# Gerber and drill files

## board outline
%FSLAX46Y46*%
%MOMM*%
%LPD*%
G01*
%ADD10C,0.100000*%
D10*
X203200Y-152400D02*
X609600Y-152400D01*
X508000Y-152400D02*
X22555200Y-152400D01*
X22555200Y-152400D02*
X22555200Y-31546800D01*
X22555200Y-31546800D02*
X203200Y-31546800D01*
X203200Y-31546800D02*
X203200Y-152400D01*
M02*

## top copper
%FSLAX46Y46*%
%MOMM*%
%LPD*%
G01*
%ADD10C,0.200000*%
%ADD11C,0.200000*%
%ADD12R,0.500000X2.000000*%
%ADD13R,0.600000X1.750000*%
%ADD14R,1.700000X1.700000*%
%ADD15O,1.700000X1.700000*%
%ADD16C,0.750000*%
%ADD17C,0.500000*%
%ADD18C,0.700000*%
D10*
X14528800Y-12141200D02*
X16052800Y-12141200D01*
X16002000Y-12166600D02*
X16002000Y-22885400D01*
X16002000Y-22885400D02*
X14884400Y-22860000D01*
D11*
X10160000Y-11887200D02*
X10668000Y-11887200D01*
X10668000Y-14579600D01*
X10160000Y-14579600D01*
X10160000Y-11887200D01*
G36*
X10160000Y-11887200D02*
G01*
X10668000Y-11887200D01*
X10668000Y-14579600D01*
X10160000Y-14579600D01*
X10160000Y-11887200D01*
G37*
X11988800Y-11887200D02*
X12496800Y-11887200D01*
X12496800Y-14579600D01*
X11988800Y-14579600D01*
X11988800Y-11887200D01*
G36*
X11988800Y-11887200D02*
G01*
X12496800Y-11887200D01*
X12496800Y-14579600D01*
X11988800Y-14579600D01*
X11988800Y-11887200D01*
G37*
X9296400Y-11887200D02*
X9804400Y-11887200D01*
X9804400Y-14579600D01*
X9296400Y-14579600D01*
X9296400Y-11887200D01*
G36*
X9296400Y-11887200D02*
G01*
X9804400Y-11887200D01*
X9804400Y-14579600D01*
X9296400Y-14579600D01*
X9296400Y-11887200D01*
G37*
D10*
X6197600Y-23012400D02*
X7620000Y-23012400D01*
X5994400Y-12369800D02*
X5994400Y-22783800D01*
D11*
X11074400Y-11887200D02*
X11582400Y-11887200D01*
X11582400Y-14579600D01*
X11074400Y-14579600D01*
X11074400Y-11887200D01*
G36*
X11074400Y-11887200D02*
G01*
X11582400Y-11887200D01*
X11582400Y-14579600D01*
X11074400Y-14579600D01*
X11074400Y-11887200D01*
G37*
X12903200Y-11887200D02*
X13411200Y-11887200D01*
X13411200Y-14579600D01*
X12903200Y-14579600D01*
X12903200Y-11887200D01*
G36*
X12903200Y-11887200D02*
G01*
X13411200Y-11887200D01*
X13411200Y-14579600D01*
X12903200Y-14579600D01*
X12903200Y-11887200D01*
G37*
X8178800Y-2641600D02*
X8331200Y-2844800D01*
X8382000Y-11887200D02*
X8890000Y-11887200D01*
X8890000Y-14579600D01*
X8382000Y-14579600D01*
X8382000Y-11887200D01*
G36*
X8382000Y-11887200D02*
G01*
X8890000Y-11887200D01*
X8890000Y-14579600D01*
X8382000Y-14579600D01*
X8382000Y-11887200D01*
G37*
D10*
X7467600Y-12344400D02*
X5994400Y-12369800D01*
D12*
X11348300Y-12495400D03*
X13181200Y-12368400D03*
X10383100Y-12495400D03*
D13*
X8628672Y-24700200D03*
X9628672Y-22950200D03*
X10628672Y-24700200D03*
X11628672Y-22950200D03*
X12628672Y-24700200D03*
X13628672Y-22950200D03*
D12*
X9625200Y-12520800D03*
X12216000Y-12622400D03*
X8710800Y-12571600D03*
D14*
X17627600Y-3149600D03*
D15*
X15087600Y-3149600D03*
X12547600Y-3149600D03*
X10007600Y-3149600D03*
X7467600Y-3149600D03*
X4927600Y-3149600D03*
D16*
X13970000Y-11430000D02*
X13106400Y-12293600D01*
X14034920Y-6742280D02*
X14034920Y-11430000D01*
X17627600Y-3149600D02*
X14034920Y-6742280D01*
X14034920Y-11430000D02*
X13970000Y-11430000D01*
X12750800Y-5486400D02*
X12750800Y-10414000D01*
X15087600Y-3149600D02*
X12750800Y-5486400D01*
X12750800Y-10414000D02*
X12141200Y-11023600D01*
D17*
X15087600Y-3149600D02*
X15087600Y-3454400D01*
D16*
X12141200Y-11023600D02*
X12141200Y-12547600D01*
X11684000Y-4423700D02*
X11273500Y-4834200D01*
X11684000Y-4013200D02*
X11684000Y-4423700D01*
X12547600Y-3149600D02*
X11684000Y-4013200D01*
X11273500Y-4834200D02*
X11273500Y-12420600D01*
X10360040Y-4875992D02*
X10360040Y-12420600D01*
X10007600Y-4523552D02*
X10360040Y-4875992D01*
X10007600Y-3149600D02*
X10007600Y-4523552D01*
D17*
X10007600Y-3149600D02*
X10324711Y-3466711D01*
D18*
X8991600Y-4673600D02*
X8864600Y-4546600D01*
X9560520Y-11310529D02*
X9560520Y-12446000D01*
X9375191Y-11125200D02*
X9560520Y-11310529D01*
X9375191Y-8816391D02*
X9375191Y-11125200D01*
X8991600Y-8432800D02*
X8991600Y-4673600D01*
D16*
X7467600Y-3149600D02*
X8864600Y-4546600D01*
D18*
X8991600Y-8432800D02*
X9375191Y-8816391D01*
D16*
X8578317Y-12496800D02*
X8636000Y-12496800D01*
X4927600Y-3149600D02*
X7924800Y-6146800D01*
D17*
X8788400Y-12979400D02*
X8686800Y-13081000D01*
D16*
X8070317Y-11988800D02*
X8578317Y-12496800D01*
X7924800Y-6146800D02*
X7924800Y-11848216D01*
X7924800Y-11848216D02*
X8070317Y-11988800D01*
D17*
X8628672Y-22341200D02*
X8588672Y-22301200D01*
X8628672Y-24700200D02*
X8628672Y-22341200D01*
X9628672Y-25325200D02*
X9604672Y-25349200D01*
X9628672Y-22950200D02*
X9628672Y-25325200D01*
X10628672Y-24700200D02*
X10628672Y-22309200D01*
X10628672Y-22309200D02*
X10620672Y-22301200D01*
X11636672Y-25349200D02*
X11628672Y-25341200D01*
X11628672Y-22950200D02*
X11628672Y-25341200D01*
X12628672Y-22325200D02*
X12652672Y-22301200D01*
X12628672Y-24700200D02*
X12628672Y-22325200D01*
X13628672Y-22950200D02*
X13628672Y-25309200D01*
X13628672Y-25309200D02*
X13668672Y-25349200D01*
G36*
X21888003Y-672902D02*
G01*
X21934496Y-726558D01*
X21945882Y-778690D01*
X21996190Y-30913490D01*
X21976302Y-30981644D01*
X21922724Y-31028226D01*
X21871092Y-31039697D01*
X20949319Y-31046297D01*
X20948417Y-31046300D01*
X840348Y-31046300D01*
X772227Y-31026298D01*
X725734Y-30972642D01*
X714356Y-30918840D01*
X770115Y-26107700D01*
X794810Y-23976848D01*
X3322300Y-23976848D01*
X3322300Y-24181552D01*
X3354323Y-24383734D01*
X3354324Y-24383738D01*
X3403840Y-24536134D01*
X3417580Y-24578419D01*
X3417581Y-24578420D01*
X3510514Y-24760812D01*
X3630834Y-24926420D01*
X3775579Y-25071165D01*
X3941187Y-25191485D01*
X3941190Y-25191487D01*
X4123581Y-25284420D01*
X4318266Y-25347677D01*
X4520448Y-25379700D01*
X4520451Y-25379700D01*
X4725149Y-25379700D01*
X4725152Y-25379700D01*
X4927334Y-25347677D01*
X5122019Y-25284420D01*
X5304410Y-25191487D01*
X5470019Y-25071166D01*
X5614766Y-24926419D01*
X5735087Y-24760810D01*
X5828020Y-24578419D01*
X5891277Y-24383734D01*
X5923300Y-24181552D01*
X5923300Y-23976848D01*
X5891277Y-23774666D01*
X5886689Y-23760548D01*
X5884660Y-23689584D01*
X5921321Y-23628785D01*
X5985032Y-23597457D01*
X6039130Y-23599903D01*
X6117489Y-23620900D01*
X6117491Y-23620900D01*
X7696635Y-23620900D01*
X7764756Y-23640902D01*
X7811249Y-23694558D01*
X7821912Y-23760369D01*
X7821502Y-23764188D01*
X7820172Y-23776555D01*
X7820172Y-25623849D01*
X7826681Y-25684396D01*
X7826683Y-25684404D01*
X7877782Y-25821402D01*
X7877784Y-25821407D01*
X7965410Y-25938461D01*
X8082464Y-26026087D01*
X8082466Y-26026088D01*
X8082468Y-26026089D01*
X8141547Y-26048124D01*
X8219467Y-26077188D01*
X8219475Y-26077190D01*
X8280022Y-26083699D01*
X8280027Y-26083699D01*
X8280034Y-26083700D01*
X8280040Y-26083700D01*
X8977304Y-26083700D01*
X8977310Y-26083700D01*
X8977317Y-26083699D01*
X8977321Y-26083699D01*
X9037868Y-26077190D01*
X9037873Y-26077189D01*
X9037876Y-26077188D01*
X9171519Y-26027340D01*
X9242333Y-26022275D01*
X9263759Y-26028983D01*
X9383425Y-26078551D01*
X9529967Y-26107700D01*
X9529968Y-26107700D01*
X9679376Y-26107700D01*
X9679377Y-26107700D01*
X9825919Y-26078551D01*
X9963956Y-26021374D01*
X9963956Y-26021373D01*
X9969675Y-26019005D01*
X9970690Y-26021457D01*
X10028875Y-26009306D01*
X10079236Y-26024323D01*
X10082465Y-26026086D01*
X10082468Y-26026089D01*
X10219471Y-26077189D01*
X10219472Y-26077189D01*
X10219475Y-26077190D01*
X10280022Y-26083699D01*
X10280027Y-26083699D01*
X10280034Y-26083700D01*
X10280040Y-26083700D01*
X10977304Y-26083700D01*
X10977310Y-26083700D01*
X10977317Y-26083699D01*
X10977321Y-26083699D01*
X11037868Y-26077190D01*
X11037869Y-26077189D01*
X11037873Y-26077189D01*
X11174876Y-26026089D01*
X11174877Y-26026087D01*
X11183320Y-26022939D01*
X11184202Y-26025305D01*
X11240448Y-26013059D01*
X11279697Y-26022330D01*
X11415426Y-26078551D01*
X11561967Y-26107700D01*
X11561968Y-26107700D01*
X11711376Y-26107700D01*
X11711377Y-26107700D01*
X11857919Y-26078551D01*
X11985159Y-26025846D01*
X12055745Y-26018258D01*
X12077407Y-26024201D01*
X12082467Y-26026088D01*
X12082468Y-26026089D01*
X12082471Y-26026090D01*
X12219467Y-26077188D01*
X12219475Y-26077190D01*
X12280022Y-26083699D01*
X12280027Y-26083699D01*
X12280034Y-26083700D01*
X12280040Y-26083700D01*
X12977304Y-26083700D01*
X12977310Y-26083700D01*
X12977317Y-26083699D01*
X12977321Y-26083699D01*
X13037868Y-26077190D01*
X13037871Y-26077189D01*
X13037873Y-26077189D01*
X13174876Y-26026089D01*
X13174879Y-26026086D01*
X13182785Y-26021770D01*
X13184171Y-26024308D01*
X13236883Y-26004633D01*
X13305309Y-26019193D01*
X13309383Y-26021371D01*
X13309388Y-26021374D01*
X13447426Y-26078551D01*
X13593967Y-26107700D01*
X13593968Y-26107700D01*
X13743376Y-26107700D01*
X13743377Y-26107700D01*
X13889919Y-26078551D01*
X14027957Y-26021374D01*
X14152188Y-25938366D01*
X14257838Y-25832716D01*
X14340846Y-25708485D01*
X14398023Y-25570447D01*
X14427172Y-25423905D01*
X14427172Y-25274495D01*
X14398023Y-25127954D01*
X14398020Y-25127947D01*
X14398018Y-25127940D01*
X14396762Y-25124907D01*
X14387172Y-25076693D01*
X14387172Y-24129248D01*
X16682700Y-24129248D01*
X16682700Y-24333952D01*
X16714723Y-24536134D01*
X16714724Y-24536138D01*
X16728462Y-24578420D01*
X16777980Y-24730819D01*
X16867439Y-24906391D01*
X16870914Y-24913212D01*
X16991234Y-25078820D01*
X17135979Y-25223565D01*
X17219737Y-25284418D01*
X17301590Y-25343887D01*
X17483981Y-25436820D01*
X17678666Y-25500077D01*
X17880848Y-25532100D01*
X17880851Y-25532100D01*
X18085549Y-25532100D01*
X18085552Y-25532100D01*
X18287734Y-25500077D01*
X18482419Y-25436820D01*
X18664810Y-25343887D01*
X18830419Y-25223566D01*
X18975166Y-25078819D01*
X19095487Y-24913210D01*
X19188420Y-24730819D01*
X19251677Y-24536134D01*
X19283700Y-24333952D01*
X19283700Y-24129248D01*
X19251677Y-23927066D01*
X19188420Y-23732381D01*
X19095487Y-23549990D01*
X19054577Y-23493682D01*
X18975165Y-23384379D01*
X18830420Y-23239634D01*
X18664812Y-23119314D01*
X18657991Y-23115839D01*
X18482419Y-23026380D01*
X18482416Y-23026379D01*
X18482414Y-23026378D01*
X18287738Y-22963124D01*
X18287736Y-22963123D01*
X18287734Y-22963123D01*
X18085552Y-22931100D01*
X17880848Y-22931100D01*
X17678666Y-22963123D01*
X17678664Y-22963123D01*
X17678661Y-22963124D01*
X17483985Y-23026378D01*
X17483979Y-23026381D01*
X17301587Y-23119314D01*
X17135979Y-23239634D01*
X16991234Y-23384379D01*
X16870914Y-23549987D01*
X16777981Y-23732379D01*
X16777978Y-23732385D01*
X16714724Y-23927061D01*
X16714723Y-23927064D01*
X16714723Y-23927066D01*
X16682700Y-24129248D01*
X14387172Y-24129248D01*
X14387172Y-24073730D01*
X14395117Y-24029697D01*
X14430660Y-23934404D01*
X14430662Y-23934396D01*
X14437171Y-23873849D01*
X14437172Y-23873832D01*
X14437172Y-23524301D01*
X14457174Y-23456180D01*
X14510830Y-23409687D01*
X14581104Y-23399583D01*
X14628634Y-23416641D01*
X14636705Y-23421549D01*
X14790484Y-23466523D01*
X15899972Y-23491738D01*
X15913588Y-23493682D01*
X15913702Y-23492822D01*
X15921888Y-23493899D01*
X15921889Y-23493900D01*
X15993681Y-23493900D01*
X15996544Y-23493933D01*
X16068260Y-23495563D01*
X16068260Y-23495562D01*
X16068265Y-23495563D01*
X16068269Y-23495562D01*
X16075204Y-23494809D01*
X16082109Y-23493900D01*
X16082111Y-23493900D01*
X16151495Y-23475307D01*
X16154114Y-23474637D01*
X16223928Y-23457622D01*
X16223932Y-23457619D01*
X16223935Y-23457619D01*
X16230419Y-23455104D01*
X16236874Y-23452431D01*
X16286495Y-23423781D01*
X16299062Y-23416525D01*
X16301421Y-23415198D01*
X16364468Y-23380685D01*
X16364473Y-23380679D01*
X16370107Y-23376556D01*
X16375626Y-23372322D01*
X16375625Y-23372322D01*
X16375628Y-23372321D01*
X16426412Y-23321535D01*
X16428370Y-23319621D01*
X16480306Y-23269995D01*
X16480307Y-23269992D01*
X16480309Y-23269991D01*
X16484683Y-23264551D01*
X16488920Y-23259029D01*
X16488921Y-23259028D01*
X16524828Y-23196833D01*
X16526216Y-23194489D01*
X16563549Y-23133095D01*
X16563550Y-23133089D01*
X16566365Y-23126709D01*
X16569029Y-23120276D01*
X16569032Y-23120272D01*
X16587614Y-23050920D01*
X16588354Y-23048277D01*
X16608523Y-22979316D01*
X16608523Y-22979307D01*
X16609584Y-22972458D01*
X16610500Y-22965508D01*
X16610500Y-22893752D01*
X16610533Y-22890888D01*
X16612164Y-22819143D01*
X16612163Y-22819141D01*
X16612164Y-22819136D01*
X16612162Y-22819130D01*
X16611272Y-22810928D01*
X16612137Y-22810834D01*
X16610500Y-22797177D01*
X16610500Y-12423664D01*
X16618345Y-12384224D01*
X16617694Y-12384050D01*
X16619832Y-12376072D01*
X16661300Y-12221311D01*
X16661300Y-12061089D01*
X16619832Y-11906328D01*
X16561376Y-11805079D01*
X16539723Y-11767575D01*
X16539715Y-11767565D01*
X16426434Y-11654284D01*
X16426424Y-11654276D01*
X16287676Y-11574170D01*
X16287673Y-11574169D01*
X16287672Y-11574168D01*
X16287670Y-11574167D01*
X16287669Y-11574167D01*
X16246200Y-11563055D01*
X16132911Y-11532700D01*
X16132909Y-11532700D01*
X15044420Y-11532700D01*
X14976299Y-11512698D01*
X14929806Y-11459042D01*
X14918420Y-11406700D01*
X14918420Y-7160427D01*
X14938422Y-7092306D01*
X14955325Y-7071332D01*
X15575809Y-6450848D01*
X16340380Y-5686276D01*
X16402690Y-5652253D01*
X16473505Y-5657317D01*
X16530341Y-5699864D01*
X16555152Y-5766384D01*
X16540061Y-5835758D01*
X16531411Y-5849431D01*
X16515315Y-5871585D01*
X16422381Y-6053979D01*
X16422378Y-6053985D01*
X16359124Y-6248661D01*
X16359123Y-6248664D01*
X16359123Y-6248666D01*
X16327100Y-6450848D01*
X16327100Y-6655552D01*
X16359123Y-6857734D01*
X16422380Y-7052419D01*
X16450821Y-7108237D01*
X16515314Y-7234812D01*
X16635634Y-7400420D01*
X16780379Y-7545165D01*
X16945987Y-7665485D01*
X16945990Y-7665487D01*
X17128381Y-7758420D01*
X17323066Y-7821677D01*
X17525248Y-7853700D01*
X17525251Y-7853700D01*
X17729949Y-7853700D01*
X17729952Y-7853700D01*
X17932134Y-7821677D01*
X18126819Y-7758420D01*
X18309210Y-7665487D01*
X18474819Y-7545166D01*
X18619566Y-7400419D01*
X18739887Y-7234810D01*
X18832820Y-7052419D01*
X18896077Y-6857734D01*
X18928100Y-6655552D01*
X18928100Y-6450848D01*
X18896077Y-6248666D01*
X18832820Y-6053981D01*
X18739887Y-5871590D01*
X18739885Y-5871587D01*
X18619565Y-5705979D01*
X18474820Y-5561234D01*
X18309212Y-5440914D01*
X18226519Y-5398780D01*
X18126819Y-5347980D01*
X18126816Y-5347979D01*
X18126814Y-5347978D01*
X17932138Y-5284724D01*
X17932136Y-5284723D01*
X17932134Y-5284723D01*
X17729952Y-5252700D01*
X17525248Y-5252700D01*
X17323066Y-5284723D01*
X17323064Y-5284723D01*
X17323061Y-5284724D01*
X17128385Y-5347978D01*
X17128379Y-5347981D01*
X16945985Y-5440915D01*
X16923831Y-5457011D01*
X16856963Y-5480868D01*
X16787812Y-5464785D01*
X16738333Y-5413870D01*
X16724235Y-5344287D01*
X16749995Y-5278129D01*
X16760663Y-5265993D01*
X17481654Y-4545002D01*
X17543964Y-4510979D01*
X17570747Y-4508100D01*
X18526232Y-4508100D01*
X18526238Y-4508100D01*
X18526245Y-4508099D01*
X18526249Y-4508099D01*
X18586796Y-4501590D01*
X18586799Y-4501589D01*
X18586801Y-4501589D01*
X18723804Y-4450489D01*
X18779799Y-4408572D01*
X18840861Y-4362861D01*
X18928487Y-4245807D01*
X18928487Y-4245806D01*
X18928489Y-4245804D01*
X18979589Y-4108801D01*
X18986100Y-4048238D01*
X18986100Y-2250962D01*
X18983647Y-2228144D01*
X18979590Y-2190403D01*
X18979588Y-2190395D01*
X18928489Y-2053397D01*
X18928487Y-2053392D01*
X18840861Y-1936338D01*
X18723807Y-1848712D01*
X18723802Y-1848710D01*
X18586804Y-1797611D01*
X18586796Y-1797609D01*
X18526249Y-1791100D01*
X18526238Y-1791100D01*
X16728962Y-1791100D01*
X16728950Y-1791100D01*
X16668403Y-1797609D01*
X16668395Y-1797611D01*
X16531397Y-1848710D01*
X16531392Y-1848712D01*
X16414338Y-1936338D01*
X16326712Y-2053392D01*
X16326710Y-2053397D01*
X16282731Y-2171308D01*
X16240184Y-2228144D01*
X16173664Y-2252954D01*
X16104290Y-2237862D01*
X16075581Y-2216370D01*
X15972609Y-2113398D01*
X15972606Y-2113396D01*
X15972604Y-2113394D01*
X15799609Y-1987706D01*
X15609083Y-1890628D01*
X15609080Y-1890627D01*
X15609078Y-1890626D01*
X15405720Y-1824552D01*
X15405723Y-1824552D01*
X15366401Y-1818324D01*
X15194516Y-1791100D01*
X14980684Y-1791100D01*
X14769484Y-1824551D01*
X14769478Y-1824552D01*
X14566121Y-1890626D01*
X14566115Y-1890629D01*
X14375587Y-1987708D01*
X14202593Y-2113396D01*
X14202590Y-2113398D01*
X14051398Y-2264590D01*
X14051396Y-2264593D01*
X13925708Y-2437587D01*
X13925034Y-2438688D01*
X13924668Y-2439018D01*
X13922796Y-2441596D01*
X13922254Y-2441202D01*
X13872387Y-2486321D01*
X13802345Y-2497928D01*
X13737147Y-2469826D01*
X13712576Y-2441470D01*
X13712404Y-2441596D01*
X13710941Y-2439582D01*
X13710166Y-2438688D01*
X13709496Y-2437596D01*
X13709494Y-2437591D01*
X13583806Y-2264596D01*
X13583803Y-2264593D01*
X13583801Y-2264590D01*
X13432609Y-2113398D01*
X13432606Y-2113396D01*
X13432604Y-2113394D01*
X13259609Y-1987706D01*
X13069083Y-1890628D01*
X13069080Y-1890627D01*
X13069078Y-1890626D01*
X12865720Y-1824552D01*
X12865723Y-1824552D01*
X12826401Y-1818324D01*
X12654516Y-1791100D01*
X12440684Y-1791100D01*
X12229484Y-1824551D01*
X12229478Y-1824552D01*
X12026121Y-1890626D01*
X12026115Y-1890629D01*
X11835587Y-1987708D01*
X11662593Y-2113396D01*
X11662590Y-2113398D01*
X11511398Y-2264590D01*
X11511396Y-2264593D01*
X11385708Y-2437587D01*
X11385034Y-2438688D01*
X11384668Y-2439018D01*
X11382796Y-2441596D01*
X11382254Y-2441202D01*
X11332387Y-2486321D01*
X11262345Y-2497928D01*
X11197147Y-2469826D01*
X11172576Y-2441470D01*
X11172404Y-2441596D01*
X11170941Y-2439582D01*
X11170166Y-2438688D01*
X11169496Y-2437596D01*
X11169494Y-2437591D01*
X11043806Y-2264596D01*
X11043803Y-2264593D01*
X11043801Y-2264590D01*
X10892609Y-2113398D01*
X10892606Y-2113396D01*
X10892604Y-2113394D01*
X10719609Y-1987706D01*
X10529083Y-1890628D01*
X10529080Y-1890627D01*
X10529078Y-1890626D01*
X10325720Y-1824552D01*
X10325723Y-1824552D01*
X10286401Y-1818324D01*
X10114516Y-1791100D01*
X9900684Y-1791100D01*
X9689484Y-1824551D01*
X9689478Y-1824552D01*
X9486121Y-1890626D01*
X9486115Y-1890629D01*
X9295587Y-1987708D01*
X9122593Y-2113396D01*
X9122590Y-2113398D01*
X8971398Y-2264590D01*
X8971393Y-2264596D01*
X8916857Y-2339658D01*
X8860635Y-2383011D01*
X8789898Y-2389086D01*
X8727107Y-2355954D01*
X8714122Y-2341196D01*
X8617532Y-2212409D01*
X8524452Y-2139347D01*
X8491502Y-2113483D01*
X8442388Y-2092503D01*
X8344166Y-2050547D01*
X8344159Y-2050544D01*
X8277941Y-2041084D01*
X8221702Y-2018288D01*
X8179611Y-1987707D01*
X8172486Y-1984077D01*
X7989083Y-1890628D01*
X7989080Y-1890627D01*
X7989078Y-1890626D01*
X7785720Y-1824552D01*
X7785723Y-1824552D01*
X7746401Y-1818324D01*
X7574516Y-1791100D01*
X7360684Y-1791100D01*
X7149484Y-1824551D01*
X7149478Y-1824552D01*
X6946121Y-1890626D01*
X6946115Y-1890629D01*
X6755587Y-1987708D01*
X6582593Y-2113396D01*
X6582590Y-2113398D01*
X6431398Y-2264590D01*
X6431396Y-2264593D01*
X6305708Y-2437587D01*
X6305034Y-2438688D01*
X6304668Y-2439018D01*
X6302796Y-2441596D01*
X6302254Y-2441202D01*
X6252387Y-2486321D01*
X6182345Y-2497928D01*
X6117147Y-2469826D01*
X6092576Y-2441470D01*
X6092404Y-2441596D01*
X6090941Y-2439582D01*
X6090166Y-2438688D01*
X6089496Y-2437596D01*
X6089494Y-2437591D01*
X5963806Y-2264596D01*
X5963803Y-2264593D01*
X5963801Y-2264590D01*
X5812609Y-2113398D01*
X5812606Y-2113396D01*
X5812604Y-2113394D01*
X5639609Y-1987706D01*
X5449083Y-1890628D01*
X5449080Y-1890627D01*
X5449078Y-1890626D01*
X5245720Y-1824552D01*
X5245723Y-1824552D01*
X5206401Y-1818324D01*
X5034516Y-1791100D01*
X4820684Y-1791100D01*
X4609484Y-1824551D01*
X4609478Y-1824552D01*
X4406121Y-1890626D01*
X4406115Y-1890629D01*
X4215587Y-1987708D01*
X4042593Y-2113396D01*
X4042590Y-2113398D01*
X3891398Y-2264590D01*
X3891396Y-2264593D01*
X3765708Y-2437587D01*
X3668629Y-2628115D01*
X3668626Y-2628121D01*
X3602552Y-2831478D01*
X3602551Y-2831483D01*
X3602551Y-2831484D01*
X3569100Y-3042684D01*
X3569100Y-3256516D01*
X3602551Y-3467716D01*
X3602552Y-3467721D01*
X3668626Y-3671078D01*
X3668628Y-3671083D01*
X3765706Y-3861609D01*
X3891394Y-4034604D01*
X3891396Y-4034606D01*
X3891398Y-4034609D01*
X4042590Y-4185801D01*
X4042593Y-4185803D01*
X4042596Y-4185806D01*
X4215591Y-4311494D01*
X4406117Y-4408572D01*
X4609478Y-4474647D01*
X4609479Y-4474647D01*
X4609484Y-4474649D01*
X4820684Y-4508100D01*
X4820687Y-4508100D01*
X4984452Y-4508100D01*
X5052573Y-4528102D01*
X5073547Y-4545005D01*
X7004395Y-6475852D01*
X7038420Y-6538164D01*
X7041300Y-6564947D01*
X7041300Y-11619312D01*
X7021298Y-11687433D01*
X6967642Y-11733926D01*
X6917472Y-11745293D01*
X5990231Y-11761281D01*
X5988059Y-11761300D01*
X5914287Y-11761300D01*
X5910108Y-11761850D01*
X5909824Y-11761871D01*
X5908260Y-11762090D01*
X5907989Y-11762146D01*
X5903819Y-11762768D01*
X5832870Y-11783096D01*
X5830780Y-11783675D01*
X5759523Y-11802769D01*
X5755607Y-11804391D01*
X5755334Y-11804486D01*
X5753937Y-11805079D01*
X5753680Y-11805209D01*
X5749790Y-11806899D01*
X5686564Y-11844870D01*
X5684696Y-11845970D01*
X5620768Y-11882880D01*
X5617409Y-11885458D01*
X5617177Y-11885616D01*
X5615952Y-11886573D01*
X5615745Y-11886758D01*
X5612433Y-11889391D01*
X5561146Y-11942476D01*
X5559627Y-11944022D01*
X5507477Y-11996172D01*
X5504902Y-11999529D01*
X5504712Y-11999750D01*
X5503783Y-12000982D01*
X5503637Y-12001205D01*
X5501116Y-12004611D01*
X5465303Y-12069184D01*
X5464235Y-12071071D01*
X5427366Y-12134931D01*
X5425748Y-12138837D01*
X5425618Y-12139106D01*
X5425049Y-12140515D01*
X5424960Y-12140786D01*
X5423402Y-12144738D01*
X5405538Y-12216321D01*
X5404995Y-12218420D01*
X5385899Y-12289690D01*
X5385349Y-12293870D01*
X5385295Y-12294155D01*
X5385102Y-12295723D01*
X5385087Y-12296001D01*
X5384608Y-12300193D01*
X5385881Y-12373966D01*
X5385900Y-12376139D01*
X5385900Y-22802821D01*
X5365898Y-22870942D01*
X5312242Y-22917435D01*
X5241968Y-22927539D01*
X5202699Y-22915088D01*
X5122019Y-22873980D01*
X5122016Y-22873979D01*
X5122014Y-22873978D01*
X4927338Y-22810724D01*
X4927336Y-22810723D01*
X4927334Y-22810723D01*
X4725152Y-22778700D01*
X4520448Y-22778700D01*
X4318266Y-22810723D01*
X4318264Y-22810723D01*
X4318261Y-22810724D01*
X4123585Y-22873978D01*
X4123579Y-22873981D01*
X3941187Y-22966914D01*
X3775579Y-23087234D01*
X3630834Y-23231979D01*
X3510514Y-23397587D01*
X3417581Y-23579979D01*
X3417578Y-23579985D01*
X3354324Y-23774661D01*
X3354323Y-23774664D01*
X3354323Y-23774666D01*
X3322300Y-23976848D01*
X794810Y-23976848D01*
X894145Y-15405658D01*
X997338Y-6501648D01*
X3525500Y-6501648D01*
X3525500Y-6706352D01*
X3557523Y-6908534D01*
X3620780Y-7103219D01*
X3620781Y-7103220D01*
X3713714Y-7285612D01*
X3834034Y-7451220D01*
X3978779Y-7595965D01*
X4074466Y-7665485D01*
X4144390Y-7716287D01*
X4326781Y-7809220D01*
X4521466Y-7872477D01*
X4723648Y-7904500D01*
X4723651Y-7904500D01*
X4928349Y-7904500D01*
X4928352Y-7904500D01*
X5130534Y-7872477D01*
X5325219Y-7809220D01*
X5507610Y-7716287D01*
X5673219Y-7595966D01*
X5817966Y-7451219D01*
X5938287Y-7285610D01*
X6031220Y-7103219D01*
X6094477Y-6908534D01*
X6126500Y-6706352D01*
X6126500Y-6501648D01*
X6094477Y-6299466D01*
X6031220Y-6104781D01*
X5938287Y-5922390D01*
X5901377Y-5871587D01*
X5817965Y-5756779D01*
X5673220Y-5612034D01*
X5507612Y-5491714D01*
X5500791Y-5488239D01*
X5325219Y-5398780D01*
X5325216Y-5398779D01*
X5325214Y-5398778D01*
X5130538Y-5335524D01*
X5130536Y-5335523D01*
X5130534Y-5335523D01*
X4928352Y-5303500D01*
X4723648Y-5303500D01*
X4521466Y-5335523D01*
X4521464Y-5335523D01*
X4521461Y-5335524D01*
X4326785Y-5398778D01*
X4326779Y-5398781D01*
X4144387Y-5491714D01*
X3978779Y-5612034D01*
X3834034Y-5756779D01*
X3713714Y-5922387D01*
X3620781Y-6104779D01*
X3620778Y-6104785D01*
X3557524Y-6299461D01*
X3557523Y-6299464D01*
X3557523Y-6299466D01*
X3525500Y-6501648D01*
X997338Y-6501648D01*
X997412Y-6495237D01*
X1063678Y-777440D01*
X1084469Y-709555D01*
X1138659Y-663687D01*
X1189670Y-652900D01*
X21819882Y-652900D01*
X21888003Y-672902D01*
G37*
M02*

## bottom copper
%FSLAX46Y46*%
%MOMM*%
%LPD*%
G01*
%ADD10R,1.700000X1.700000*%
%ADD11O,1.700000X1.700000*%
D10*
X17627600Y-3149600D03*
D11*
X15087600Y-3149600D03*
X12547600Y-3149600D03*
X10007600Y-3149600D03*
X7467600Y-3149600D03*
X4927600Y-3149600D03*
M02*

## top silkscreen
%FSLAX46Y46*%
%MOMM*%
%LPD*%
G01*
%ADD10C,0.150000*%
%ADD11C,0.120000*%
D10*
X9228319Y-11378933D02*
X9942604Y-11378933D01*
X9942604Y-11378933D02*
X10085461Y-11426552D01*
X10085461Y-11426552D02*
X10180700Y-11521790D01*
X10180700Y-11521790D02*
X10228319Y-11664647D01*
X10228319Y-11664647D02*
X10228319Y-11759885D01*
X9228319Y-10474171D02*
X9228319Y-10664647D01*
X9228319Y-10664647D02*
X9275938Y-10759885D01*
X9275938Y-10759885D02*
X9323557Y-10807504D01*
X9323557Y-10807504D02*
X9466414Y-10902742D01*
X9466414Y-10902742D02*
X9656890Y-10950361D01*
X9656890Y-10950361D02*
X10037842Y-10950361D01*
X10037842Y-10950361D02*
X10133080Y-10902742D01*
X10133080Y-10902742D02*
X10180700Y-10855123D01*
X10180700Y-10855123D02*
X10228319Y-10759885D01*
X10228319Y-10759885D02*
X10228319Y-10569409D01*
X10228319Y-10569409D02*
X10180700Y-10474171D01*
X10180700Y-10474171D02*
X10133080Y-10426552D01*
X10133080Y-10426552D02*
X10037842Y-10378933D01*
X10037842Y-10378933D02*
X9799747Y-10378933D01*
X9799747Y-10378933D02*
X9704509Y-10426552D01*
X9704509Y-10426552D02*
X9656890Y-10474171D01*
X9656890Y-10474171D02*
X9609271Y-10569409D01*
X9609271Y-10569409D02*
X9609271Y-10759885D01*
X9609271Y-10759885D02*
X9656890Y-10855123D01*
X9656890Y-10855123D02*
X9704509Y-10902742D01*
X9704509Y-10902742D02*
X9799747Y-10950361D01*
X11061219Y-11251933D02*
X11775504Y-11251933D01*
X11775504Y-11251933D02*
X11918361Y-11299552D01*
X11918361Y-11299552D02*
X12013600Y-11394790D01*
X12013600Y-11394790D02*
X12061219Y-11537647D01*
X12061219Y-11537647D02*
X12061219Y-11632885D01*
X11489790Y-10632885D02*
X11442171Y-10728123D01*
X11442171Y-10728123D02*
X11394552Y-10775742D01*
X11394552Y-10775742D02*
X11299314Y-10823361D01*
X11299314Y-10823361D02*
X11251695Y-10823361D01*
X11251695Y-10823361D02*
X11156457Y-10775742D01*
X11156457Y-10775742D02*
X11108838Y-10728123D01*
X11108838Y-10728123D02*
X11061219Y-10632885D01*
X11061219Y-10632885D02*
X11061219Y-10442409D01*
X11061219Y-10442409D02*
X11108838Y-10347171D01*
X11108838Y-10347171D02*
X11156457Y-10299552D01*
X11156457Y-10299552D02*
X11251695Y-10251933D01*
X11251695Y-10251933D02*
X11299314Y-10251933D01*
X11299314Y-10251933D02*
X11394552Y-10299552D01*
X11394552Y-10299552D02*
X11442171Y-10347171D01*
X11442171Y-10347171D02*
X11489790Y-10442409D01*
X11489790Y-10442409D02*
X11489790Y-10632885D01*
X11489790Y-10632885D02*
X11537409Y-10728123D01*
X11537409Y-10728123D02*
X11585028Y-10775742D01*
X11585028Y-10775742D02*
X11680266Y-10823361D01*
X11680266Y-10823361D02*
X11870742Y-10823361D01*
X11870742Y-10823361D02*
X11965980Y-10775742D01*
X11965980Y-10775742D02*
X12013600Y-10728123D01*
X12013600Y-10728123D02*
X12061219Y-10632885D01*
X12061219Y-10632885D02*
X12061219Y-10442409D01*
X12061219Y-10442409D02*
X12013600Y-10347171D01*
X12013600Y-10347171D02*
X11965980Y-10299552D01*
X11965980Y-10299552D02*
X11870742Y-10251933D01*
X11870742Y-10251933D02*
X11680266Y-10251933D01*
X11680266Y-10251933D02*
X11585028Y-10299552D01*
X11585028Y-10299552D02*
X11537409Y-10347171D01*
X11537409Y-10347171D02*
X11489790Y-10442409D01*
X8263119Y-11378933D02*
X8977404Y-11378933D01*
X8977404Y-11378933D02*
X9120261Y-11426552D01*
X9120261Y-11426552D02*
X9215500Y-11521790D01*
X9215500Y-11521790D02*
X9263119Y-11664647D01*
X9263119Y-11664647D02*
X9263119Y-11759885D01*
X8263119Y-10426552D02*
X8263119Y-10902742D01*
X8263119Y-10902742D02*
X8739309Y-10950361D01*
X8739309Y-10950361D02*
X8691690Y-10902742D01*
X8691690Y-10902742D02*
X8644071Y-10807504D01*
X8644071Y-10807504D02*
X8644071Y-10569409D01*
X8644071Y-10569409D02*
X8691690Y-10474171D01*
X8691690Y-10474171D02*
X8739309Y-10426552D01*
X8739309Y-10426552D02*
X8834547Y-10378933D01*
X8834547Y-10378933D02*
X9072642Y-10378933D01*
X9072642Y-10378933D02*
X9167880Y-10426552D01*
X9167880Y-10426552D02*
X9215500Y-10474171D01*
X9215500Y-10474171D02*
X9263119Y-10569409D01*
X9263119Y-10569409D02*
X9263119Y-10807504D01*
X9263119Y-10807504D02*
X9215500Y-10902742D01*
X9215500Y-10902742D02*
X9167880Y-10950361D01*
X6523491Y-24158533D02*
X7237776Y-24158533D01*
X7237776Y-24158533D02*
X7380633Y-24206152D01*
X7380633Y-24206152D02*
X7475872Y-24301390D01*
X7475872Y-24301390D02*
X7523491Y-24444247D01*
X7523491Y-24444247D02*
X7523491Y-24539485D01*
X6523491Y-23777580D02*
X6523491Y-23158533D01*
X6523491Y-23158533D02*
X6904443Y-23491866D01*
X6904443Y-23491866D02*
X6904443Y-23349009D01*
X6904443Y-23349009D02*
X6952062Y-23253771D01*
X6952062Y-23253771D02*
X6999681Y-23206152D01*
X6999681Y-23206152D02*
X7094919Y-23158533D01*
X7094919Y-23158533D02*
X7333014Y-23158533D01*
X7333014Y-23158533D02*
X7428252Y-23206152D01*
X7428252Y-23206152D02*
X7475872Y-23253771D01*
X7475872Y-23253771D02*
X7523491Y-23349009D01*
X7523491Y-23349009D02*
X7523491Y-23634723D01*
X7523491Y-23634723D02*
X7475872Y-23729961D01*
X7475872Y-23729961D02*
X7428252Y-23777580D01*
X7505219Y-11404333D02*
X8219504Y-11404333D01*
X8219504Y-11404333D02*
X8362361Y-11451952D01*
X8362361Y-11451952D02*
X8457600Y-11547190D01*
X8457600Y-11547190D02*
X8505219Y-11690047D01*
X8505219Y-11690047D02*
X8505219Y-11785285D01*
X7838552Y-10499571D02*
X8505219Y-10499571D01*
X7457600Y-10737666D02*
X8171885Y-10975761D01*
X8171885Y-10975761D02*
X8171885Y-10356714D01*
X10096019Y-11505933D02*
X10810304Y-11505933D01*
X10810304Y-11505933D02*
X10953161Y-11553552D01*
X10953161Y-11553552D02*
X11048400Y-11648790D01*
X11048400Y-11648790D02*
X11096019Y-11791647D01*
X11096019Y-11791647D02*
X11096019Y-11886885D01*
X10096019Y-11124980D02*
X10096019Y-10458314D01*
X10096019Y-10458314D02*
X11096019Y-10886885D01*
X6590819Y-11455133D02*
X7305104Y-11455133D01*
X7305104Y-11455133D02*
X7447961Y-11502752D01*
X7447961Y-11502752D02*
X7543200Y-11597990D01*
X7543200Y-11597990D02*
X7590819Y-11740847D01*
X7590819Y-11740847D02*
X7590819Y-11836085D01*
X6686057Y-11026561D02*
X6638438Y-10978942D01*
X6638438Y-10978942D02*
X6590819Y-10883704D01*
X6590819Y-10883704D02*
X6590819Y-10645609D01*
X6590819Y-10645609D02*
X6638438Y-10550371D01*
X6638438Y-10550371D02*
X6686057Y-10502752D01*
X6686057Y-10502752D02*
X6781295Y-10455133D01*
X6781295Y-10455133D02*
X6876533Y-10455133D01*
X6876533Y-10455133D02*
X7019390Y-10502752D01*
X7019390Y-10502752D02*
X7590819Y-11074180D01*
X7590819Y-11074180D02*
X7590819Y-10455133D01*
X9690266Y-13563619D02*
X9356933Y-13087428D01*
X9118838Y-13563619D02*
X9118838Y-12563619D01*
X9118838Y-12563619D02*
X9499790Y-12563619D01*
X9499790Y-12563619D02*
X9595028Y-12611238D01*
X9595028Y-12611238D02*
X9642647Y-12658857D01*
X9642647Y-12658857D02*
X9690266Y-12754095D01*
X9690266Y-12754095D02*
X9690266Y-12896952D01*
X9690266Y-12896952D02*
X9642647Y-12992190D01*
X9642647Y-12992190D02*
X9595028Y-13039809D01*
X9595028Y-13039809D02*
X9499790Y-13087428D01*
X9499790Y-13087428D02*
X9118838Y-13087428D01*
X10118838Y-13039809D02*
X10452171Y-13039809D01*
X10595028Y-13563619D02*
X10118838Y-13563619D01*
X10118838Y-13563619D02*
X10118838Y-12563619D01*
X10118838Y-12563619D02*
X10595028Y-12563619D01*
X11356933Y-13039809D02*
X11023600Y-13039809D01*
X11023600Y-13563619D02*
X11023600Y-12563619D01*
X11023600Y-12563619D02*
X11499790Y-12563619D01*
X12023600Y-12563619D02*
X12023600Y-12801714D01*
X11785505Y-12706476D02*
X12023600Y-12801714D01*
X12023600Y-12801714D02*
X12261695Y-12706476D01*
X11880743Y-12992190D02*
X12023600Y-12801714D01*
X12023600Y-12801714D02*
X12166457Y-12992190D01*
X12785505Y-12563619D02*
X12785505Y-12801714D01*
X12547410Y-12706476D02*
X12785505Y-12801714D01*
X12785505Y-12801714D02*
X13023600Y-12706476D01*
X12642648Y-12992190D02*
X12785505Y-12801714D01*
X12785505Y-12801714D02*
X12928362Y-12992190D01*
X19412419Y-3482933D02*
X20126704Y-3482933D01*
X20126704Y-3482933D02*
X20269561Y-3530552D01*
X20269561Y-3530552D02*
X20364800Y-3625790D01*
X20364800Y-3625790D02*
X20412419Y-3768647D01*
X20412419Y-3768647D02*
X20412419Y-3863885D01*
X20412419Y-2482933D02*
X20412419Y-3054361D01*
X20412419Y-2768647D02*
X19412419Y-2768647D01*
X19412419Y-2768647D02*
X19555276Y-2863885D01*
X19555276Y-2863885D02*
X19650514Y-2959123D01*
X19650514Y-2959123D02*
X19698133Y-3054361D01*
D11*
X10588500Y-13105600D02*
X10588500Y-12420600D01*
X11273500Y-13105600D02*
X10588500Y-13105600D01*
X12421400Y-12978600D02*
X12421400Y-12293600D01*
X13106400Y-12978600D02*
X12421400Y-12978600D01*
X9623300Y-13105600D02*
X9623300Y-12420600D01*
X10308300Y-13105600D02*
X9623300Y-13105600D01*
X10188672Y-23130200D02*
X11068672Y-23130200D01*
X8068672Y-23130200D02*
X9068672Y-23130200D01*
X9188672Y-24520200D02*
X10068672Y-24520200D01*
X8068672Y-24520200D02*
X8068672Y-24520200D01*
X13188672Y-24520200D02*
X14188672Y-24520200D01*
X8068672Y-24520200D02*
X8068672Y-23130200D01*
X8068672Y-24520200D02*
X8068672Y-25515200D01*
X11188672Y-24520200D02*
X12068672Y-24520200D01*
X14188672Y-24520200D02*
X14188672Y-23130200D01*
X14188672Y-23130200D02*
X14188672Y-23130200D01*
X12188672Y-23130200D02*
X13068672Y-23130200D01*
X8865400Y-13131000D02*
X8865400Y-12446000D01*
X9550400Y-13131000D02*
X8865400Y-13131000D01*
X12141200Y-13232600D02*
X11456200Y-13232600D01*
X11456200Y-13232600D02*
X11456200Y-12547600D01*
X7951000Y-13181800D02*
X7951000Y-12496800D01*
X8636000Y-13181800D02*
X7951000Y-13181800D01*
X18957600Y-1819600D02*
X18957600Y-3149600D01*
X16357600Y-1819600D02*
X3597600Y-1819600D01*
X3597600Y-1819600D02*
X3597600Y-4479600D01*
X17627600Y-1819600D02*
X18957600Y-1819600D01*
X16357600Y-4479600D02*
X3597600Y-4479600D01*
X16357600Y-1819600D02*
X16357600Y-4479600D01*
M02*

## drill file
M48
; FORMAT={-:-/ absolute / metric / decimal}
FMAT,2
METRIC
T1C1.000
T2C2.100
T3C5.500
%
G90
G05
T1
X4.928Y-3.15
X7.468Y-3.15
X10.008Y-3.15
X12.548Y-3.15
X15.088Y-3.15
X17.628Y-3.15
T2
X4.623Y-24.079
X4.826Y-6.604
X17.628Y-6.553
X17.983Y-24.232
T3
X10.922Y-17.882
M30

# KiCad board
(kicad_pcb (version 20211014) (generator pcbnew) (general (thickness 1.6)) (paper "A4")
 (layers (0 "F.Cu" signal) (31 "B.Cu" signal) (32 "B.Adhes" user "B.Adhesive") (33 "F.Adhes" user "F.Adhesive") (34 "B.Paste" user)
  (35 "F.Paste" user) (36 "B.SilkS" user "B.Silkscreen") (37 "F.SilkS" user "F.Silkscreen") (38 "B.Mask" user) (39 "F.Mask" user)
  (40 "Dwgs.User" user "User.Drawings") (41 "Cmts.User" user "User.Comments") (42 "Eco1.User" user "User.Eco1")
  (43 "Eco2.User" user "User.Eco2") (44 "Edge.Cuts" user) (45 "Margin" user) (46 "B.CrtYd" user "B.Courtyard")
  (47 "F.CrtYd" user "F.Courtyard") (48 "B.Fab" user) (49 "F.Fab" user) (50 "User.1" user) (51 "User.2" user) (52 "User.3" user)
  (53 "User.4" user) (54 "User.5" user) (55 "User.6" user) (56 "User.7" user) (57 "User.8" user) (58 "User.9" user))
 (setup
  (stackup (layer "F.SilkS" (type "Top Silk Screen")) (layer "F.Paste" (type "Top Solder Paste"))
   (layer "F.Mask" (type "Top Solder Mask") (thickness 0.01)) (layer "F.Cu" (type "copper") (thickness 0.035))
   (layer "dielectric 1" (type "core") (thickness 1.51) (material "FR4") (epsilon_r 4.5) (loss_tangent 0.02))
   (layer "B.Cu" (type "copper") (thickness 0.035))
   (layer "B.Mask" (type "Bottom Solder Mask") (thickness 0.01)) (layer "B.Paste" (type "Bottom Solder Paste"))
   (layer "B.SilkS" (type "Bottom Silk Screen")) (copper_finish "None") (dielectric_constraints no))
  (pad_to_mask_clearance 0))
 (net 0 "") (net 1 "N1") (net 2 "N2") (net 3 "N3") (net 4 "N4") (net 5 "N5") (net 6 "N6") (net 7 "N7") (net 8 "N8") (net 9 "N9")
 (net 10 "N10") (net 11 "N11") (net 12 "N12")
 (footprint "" (layer "F.Cu") (at 17.9832 24.2316)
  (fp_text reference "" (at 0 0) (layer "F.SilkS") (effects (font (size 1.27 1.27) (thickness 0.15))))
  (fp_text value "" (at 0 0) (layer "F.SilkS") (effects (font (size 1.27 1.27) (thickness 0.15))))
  (pad "" np_thru_hole circle (at 0 0) (size 2.1 2.1) (drill 2.1) (layers *.Cu *.Mask)))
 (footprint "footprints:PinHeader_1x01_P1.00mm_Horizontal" (layer "F.Cu") (at 11.2735 12.4206 90)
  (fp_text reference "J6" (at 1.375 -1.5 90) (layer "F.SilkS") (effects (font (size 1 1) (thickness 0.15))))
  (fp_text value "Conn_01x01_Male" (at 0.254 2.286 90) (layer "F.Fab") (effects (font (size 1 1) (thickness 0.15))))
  (fp_line (start -0.685 -0.685) (end 0 -0.685) (layer "F.SilkS") (width 0.12))
  (fp_line (start -0.685 0) (end -0.685 -0.685) (layer "F.SilkS") (width 0.12))
  (pad "1" smd rect (at 0 0 90) (size 2 0.5) (drill (offset -0.0748 0.0748)) (layers "F.Cu" "F.Paste" "F.Mask") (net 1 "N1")))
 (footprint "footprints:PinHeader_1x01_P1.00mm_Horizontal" (layer "F.Cu") (at 13.1064 12.2936 90)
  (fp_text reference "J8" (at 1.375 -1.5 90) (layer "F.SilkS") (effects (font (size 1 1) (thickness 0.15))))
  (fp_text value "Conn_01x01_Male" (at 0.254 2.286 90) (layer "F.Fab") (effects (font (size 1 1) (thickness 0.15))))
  (fp_line (start -0.685 -0.685) (end 0 -0.685) (layer "F.SilkS") (width 0.12))
  (fp_line (start -0.685 0) (end -0.685 -0.685) (layer "F.SilkS") (width 0.12))
  (pad "1" smd rect (at 0 0 90) (size 2 0.5) (drill (offset -0.0748 0.0748)) (layers "F.Cu" "F.Paste" "F.Mask") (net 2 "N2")))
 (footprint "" (layer "F.Cu") (at 17.6276 6.5532)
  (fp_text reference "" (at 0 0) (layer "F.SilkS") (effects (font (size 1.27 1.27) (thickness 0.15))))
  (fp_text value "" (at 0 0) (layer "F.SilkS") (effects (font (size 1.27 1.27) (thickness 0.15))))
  (pad "" np_thru_hole circle (at 0 0) (size 2.1 2.1) (drill 2.1) (layers *.Cu *.Mask)))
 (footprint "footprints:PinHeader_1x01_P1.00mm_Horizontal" (layer "F.Cu") (at 10.3083 12.4206 90)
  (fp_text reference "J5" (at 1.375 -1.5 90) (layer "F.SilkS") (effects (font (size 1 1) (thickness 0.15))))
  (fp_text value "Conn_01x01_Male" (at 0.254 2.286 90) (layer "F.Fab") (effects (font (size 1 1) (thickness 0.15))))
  (fp_line (start -0.685 -0.685) (end 0 -0.685) (layer "F.SilkS") (width 0.12))
  (fp_line (start -0.685 0) (end -0.685 -0.685) (layer "F.SilkS") (width 0.12))
  (pad "1" smd rect (at 0 0 90) (size 2 0.5) (drill (offset -0.0748 0.0748)) (layers "F.Cu" "F.Paste" "F.Mask") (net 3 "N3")))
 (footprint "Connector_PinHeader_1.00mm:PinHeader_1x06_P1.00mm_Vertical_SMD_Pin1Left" (layer "F.Cu") (at 11.128672 23.8252 90)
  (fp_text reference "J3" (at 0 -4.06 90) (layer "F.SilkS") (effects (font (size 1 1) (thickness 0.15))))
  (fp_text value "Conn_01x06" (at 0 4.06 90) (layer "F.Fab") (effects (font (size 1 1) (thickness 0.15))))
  (fp_line (start 0.695 -0.94) (end 0.695 -0.06) (layer "F.SilkS") (width 0.12))
  (fp_line (start 0.695 -3.06) (end 0.695 -2.06) (layer "F.SilkS") (width 0.12))
  (fp_line (start -0.695 -1.94) (end -0.695 -1.06) (layer "F.SilkS") (width 0.12))
  (fp_line (start -0.695 -3.06) (end -0.695 -3.06) (layer "F.SilkS") (width 0.12))
  (fp_line (start -0.695 2.06) (end -0.695 3.06) (layer "F.SilkS") (width 0.12))
  (fp_line (start -0.695 -3.06) (end 0.695 -3.06) (layer "F.SilkS") (width 0.12))
  (fp_line (start -0.695 -3.06) (end -1.69 -3.06) (layer "F.SilkS") (width 0.12))
  (fp_line (start -0.695 0.06) (end -0.695 0.94) (layer "F.SilkS") (width 0.12))
  (fp_line (start -0.695 3.06) (end 0.695 3.06) (layer "F.SilkS") (width 0.12))
  (fp_line (start 0.695 3.06) (end 0.695 3.06) (layer "F.SilkS") (width 0.12))
  (fp_line (start 0.695 1.06) (end 0.695 1.94) (layer "F.SilkS") (width 0.12))
  (pad "1" smd rect (at -0.875 -2.5 90) (size 1.75 0.6) (layers "F.Cu" "F.Paste" "F.Mask") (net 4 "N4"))
  (pad "2" smd rect (at 0.875 -1.5 90) (size 1.75 0.6) (layers "F.Cu" "F.Paste" "F.Mask") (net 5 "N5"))
  (pad "3" smd rect (at -0.875 -0.5 90) (size 1.75 0.6) (layers "F.Cu" "F.Paste" "F.Mask") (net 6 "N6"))
  (pad "4" smd rect (at 0.875 0.5 90) (size 1.75 0.6) (layers "F.Cu" "F.Paste" "F.Mask") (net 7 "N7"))
  (pad "5" smd rect (at -0.875 1.5 90) (size 1.75 0.6) (layers "F.Cu" "F.Paste" "F.Mask") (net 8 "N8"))
  (pad "6" smd rect (at 0.875 2.5 90) (size 1.75 0.6) (layers "F.Cu" "F.Paste" "F.Mask") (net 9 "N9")))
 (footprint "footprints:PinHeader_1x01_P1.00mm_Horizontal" (layer "F.Cu") (at 9.5504 12.446 90)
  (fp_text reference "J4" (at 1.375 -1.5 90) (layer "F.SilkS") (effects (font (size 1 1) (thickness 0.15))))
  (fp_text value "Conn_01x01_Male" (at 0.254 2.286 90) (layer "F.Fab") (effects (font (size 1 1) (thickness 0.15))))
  (fp_line (start -0.685 -0.685) (end 0 -0.685) (layer "F.SilkS") (width 0.12))
  (fp_line (start -0.685 0) (end -0.685 -0.685) (layer "F.SilkS") (width 0.12))
  (pad "1" smd rect (at 0 0 90) (size 2 0.5) (drill (offset -0.0748 0.0748)) (layers "F.Cu" "F.Paste" "F.Mask") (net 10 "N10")))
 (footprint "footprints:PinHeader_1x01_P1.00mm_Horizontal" (layer "F.Cu") (at 12.1412 12.5476 90)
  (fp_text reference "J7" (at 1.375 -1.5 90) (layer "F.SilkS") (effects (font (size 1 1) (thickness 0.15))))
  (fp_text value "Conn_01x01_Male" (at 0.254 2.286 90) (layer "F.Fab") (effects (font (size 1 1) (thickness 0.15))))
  (fp_line (start -0.685 0) (end -0.685 -0.685) (layer "F.SilkS") (width 0.12))
  (fp_line (start -0.685 -0.685) (end 0 -0.685) (layer "F.SilkS") (width 0.12))
  (pad "1" smd rect (at 0 0 90) (size 2 0.5) (drill (offset -0.0748 0.0748)) (layers "F.Cu" "F.Paste" "F.Mask") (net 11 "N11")))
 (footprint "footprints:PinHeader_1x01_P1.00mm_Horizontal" (layer "F.Cu") (at 8.636 12.4968 90)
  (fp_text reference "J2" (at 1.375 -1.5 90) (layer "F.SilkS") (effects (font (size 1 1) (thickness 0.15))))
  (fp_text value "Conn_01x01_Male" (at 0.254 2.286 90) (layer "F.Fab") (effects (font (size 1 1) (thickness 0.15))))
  (fp_line (start -0.685 -0.685) (end 0 -0.685) (layer "F.SilkS") (width 0.12))
  (fp_line (start -0.685 0) (end -0.685 -0.685) (layer "F.SilkS") (width 0.12))
  (pad "1" smd rect (at 0 0 90) (size 2 0.5) (drill (offset -0.0748 0.0748)) (layers "F.Cu" "F.Paste" "F.Mask") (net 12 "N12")))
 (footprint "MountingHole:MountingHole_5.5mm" (layer "F.Cu") (at 10.922 17.8816)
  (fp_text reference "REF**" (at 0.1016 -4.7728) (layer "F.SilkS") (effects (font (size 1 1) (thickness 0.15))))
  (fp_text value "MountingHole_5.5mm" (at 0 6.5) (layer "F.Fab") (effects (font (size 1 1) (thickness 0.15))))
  (pad "" np_thru_hole circle (at 0 0) (size 5.5 5.5) (drill 5.5) (layers *.Cu *.Mask)))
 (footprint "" (layer "F.Cu") (at 4.6228 24.0792)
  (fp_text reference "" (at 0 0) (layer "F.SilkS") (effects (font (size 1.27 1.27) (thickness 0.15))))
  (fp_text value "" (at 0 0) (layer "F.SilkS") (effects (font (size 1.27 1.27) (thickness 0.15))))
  (pad "" np_thru_hole circle (at 0 0) (size 2.1 2.1) (drill 2.1) (layers *.Cu *.Mask)))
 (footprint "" (layer "F.Cu") (at 4.826 6.604)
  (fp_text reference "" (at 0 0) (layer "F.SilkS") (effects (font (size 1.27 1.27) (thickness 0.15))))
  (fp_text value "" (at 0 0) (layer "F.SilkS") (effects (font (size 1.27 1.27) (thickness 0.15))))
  (pad "" np_thru_hole circle (at 0 0) (size 2.1 2.1) (drill 2.1) (layers *.Cu *.Mask)))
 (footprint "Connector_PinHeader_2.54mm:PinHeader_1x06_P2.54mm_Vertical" (layer "F.Cu") (at 17.6276 3.1496 -90)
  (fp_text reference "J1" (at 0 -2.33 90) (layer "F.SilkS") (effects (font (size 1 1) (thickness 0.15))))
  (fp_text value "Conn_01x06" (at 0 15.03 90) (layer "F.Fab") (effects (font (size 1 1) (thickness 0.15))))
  (fp_line (start -1.33 -1.33) (end 0 -1.33) (layer "F.SilkS") (width 0.12))
  (fp_line (start -1.33 1.27) (end -1.33 14.03) (layer "F.SilkS") (width 0.12))
  (fp_line (start -1.33 14.03) (end 1.33 14.03) (layer "F.SilkS") (width 0.12))
  (fp_line (start -1.33 0) (end -1.33 -1.33) (layer "F.SilkS") (width 0.12))
  (fp_line (start 1.33 1.27) (end 1.33 14.03) (layer "F.SilkS") (width 0.12))
  (fp_line (start -1.33 1.27) (end 1.33 1.27) (layer "F.SilkS") (width 0.12))
  (pad "1" thru_hole rect (at 0 0 270) (size 1.7 1.7) (drill 1) (layers *.Cu *.Mask) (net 2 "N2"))
  (pad "2" thru_hole oval (at 0 2.54 270) (size 1.7 1.7) (drill 1) (layers *.Cu *.Mask) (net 11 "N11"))
  (pad "3" thru_hole oval (at 0 5.08 270) (size 1.7 1.7) (drill 1) (layers *.Cu *.Mask) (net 1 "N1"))
  (pad "4" thru_hole oval (at 0 7.62 270) (size 1.7 1.7) (drill 1) (layers *.Cu *.Mask) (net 3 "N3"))
  (pad "5" thru_hole oval (at 0 10.16 270) (size 1.7 1.7) (drill 1) (layers *.Cu *.Mask) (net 10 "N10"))
  (pad "6" thru_hole oval (at 0 12.7 270) (size 1.7 1.7) (drill 1) (layers *.Cu *.Mask) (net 12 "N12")))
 (gr_line (start 14.5288 12.1412) (end 16.0528 12.1412) (layer "F.Cu") (width 0.2))
 (gr_line (start 16.002 12.1666) (end 16.002 22.8854) (layer "F.Cu") (width 0.2))
 (gr_line (start 16.002 22.8854) (end 14.8844 22.86) (layer "F.Cu") (width 0.2))
 (gr_rect (start 10.668 11.8872) (end 10.16 14.5796) (layer "F.Cu") (width 0.2) (fill solid))
 (gr_rect (start 12.4968 11.8872) (end 11.9888 14.5796) (layer "F.Cu") (width 0.2) (fill solid))
 (gr_rect (start 9.8044 11.8872) (end 9.2964 14.5796) (layer "F.Cu") (width 0.2) (fill solid))
 (gr_line (start 6.1976 23.0124) (end 7.62 23.0124) (layer "F.Cu") (width 0.2))
 (gr_line (start 5.9944 12.3698) (end 5.9944 22.7838) (layer "F.Cu") (width 0.2))
 (gr_rect (start 11.5824 11.8872) (end 11.0744 14.5796) (layer "F.Cu") (width 0.2) (fill solid))
 (gr_rect (start 13.4112 11.8872) (end 12.9032 14.5796) (layer "F.Cu") (width 0.2) (fill solid))
 (gr_line (start 8.1788 2.6416) (end 8.3312 2.8448) (layer "F.Cu") (width 0.2))
 (gr_rect (start 8.89 11.8872) (end 8.382 14.5796) (layer "F.Cu") (width 0.2) (fill solid))
 (gr_line (start 7.4676 12.3444) (end 5.9944 12.3698) (layer "F.Cu") (width 0.2))
 (gr_line (start 0.2032 0.1524) (end 0.6096 0.1524) (layer "Edge.Cuts") (width 0.1))
 (gr_line (start 0.508 0.1524) (end 22.5552 0.1524) (layer "Edge.Cuts") (width 0.1))
 (gr_line (start 22.5552 0.1524) (end 22.5552 31.5468) (layer "Edge.Cuts") (width 0.1))
 (gr_line (start 22.5552 31.5468) (end 0.2032 31.5468) (layer "Edge.Cuts") (width 0.1))
 (gr_line (start 0.2032 31.5468) (end 0.2032 0.1524) (layer "Edge.Cuts") (width 0.1))
 (segment (start 13.97 11.43) (end 13.1064 12.2936) (width 0.75) (layer "F.Cu") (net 2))
 (segment (start 14.03492 6.74228) (end 14.03492 11.43) (width 0.75) (layer "F.Cu") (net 2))
 (segment (start 17.6276 3.1496) (end 14.03492 6.74228) (width 0.75) (layer "F.Cu") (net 2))
 (segment (start 14.03492 11.43) (end 13.97 11.43) (width 0.75) (layer "F.Cu") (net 2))
 (segment (start 12.7508 5.4864) (end 12.7508 10.414) (width 0.75) (layer "F.Cu") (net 11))
 (segment (start 15.0876 3.1496) (end 12.7508 5.4864) (width 0.75) (layer "F.Cu") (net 11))
 (segment (start 12.7508 10.414) (end 12.1412 11.0236) (width 0.75) (layer "F.Cu") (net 11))
 (segment (start 15.0876 3.1496) (end 15.0876 3.4544) (width 0.5) (layer "F.Cu") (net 11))
 (segment (start 12.1412 11.0236) (end 12.1412 12.5476) (width 0.75) (layer "F.Cu") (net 11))
 (segment (start 11.684 4.4237) (end 11.2735 4.8342) (width 0.75) (layer "F.Cu") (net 1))
 (segment (start 11.684 4.0132) (end 11.684 4.4237) (width 0.75) (layer "F.Cu") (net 1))
 (segment (start 12.5476 3.1496) (end 11.684 4.0132) (width 0.75) (layer "F.Cu") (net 1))
 (segment (start 11.2735 4.8342) (end 11.2735 12.4206) (width 0.75) (layer "F.Cu") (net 1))
 (segment (start 10.36004 4.875992) (end 10.36004 12.4206) (width 0.75) (layer "F.Cu") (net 3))
 (segment (start 10.0076 4.523552) (end 10.36004 4.875992) (width 0.75) (layer "F.Cu") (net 3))
 (segment (start 10.0076 3.1496) (end 10.0076 4.523552) (width 0.75) (layer "F.Cu") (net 3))
 (segment (start 10.0076 3.1496) (end 10.324711 3.466711) (width 0.5) (layer "F.Cu") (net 3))
 (segment (start 8.9916 4.6736) (end 8.8646 4.5466) (width 0.7) (layer "F.Cu") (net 10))
 (segment (start 9.56052 11.310529) (end 9.56052 12.446) (width 0.7) (layer "F.Cu") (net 10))
 (segment (start 9.375191 11.1252) (end 9.56052 11.310529) (width 0.7) (layer "F.Cu") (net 10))
 (segment (start 9.375191 8.816391) (end 9.375191 11.1252) (width 0.7) (layer "F.Cu") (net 10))
 (segment (start 8.9916 8.4328) (end 8.9916 4.6736) (width 0.7) (layer "F.Cu") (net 10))
 (segment (start 7.4676 3.1496) (end 8.8646 4.5466) (width 0.75) (layer "F.Cu") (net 10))
 (segment (start 8.9916 8.4328) (end 9.375191 8.816391) (width 0.7) (layer "F.Cu") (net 10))
 (segment (start 8.578317 12.4968) (end 8.636 12.4968) (width 0.75) (layer "F.Cu") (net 12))
 (segment (start 4.9276 3.1496) (end 7.9248 6.1468) (width 0.75) (layer "F.Cu") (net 12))
 (segment (start 8.7884 12.9794) (end 8.6868 13.081) (width 0.5) (layer "F.Cu") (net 12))
 (segment (start 8.070317 11.9888) (end 8.578317 12.4968) (width 0.75) (layer "F.Cu") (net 12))
 (segment (start 7.9248 6.1468) (end 7.9248 11.848216) (width 0.75) (layer "F.Cu") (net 12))
 (segment (start 7.9248 11.848216) (end 8.070317 11.9888) (width 0.75) (layer "F.Cu") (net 12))
 (segment (start 8.628672 22.3412) (end 8.588672 22.3012) (width 0.5) (layer "F.Cu") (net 4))
 (segment (start 8.628672 24.7002) (end 8.628672 22.3412) (width 0.5) (layer "F.Cu") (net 4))
 (segment (start 9.628672 25.3252) (end 9.604672 25.3492) (width 0.5) (layer "F.Cu") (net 5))
 (segment (start 9.628672 22.9502) (end 9.628672 25.3252) (width 0.5) (layer "F.Cu") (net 5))
 (segment (start 10.628672 24.7002) (end 10.628672 22.3092) (width 0.5) (layer "F.Cu") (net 6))
 (segment (start 10.628672 22.3092) (end 10.620672 22.3012) (width 0.5) (layer "F.Cu") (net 6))
 (segment (start 11.636672 25.3492) (end 11.628672 25.3412) (width 0.5) (layer "F.Cu") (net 7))
 (segment (start 11.628672 22.9502) (end 11.628672 25.3412) (width 0.5) (layer "F.Cu") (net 7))
 (segment (start 12.628672 22.3252) (end 12.652672 22.3012) (width 0.5) (layer "F.Cu") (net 8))
 (segment (start 12.628672 24.7002) (end 12.628672 22.3252) (width 0.5) (layer "F.Cu") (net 8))
 (segment (start 13.628672 22.9502) (end 13.628672 25.3092) (width 0.5) (layer "F.Cu") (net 9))
 (segment (start 13.628672 25.3092) (end 13.668672 25.3492) (width 0.5) (layer "F.Cu") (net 9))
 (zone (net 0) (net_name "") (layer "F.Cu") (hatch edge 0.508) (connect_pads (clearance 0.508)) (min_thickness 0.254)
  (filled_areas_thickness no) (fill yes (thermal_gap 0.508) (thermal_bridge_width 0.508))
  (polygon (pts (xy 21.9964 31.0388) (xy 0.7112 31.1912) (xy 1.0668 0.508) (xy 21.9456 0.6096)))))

